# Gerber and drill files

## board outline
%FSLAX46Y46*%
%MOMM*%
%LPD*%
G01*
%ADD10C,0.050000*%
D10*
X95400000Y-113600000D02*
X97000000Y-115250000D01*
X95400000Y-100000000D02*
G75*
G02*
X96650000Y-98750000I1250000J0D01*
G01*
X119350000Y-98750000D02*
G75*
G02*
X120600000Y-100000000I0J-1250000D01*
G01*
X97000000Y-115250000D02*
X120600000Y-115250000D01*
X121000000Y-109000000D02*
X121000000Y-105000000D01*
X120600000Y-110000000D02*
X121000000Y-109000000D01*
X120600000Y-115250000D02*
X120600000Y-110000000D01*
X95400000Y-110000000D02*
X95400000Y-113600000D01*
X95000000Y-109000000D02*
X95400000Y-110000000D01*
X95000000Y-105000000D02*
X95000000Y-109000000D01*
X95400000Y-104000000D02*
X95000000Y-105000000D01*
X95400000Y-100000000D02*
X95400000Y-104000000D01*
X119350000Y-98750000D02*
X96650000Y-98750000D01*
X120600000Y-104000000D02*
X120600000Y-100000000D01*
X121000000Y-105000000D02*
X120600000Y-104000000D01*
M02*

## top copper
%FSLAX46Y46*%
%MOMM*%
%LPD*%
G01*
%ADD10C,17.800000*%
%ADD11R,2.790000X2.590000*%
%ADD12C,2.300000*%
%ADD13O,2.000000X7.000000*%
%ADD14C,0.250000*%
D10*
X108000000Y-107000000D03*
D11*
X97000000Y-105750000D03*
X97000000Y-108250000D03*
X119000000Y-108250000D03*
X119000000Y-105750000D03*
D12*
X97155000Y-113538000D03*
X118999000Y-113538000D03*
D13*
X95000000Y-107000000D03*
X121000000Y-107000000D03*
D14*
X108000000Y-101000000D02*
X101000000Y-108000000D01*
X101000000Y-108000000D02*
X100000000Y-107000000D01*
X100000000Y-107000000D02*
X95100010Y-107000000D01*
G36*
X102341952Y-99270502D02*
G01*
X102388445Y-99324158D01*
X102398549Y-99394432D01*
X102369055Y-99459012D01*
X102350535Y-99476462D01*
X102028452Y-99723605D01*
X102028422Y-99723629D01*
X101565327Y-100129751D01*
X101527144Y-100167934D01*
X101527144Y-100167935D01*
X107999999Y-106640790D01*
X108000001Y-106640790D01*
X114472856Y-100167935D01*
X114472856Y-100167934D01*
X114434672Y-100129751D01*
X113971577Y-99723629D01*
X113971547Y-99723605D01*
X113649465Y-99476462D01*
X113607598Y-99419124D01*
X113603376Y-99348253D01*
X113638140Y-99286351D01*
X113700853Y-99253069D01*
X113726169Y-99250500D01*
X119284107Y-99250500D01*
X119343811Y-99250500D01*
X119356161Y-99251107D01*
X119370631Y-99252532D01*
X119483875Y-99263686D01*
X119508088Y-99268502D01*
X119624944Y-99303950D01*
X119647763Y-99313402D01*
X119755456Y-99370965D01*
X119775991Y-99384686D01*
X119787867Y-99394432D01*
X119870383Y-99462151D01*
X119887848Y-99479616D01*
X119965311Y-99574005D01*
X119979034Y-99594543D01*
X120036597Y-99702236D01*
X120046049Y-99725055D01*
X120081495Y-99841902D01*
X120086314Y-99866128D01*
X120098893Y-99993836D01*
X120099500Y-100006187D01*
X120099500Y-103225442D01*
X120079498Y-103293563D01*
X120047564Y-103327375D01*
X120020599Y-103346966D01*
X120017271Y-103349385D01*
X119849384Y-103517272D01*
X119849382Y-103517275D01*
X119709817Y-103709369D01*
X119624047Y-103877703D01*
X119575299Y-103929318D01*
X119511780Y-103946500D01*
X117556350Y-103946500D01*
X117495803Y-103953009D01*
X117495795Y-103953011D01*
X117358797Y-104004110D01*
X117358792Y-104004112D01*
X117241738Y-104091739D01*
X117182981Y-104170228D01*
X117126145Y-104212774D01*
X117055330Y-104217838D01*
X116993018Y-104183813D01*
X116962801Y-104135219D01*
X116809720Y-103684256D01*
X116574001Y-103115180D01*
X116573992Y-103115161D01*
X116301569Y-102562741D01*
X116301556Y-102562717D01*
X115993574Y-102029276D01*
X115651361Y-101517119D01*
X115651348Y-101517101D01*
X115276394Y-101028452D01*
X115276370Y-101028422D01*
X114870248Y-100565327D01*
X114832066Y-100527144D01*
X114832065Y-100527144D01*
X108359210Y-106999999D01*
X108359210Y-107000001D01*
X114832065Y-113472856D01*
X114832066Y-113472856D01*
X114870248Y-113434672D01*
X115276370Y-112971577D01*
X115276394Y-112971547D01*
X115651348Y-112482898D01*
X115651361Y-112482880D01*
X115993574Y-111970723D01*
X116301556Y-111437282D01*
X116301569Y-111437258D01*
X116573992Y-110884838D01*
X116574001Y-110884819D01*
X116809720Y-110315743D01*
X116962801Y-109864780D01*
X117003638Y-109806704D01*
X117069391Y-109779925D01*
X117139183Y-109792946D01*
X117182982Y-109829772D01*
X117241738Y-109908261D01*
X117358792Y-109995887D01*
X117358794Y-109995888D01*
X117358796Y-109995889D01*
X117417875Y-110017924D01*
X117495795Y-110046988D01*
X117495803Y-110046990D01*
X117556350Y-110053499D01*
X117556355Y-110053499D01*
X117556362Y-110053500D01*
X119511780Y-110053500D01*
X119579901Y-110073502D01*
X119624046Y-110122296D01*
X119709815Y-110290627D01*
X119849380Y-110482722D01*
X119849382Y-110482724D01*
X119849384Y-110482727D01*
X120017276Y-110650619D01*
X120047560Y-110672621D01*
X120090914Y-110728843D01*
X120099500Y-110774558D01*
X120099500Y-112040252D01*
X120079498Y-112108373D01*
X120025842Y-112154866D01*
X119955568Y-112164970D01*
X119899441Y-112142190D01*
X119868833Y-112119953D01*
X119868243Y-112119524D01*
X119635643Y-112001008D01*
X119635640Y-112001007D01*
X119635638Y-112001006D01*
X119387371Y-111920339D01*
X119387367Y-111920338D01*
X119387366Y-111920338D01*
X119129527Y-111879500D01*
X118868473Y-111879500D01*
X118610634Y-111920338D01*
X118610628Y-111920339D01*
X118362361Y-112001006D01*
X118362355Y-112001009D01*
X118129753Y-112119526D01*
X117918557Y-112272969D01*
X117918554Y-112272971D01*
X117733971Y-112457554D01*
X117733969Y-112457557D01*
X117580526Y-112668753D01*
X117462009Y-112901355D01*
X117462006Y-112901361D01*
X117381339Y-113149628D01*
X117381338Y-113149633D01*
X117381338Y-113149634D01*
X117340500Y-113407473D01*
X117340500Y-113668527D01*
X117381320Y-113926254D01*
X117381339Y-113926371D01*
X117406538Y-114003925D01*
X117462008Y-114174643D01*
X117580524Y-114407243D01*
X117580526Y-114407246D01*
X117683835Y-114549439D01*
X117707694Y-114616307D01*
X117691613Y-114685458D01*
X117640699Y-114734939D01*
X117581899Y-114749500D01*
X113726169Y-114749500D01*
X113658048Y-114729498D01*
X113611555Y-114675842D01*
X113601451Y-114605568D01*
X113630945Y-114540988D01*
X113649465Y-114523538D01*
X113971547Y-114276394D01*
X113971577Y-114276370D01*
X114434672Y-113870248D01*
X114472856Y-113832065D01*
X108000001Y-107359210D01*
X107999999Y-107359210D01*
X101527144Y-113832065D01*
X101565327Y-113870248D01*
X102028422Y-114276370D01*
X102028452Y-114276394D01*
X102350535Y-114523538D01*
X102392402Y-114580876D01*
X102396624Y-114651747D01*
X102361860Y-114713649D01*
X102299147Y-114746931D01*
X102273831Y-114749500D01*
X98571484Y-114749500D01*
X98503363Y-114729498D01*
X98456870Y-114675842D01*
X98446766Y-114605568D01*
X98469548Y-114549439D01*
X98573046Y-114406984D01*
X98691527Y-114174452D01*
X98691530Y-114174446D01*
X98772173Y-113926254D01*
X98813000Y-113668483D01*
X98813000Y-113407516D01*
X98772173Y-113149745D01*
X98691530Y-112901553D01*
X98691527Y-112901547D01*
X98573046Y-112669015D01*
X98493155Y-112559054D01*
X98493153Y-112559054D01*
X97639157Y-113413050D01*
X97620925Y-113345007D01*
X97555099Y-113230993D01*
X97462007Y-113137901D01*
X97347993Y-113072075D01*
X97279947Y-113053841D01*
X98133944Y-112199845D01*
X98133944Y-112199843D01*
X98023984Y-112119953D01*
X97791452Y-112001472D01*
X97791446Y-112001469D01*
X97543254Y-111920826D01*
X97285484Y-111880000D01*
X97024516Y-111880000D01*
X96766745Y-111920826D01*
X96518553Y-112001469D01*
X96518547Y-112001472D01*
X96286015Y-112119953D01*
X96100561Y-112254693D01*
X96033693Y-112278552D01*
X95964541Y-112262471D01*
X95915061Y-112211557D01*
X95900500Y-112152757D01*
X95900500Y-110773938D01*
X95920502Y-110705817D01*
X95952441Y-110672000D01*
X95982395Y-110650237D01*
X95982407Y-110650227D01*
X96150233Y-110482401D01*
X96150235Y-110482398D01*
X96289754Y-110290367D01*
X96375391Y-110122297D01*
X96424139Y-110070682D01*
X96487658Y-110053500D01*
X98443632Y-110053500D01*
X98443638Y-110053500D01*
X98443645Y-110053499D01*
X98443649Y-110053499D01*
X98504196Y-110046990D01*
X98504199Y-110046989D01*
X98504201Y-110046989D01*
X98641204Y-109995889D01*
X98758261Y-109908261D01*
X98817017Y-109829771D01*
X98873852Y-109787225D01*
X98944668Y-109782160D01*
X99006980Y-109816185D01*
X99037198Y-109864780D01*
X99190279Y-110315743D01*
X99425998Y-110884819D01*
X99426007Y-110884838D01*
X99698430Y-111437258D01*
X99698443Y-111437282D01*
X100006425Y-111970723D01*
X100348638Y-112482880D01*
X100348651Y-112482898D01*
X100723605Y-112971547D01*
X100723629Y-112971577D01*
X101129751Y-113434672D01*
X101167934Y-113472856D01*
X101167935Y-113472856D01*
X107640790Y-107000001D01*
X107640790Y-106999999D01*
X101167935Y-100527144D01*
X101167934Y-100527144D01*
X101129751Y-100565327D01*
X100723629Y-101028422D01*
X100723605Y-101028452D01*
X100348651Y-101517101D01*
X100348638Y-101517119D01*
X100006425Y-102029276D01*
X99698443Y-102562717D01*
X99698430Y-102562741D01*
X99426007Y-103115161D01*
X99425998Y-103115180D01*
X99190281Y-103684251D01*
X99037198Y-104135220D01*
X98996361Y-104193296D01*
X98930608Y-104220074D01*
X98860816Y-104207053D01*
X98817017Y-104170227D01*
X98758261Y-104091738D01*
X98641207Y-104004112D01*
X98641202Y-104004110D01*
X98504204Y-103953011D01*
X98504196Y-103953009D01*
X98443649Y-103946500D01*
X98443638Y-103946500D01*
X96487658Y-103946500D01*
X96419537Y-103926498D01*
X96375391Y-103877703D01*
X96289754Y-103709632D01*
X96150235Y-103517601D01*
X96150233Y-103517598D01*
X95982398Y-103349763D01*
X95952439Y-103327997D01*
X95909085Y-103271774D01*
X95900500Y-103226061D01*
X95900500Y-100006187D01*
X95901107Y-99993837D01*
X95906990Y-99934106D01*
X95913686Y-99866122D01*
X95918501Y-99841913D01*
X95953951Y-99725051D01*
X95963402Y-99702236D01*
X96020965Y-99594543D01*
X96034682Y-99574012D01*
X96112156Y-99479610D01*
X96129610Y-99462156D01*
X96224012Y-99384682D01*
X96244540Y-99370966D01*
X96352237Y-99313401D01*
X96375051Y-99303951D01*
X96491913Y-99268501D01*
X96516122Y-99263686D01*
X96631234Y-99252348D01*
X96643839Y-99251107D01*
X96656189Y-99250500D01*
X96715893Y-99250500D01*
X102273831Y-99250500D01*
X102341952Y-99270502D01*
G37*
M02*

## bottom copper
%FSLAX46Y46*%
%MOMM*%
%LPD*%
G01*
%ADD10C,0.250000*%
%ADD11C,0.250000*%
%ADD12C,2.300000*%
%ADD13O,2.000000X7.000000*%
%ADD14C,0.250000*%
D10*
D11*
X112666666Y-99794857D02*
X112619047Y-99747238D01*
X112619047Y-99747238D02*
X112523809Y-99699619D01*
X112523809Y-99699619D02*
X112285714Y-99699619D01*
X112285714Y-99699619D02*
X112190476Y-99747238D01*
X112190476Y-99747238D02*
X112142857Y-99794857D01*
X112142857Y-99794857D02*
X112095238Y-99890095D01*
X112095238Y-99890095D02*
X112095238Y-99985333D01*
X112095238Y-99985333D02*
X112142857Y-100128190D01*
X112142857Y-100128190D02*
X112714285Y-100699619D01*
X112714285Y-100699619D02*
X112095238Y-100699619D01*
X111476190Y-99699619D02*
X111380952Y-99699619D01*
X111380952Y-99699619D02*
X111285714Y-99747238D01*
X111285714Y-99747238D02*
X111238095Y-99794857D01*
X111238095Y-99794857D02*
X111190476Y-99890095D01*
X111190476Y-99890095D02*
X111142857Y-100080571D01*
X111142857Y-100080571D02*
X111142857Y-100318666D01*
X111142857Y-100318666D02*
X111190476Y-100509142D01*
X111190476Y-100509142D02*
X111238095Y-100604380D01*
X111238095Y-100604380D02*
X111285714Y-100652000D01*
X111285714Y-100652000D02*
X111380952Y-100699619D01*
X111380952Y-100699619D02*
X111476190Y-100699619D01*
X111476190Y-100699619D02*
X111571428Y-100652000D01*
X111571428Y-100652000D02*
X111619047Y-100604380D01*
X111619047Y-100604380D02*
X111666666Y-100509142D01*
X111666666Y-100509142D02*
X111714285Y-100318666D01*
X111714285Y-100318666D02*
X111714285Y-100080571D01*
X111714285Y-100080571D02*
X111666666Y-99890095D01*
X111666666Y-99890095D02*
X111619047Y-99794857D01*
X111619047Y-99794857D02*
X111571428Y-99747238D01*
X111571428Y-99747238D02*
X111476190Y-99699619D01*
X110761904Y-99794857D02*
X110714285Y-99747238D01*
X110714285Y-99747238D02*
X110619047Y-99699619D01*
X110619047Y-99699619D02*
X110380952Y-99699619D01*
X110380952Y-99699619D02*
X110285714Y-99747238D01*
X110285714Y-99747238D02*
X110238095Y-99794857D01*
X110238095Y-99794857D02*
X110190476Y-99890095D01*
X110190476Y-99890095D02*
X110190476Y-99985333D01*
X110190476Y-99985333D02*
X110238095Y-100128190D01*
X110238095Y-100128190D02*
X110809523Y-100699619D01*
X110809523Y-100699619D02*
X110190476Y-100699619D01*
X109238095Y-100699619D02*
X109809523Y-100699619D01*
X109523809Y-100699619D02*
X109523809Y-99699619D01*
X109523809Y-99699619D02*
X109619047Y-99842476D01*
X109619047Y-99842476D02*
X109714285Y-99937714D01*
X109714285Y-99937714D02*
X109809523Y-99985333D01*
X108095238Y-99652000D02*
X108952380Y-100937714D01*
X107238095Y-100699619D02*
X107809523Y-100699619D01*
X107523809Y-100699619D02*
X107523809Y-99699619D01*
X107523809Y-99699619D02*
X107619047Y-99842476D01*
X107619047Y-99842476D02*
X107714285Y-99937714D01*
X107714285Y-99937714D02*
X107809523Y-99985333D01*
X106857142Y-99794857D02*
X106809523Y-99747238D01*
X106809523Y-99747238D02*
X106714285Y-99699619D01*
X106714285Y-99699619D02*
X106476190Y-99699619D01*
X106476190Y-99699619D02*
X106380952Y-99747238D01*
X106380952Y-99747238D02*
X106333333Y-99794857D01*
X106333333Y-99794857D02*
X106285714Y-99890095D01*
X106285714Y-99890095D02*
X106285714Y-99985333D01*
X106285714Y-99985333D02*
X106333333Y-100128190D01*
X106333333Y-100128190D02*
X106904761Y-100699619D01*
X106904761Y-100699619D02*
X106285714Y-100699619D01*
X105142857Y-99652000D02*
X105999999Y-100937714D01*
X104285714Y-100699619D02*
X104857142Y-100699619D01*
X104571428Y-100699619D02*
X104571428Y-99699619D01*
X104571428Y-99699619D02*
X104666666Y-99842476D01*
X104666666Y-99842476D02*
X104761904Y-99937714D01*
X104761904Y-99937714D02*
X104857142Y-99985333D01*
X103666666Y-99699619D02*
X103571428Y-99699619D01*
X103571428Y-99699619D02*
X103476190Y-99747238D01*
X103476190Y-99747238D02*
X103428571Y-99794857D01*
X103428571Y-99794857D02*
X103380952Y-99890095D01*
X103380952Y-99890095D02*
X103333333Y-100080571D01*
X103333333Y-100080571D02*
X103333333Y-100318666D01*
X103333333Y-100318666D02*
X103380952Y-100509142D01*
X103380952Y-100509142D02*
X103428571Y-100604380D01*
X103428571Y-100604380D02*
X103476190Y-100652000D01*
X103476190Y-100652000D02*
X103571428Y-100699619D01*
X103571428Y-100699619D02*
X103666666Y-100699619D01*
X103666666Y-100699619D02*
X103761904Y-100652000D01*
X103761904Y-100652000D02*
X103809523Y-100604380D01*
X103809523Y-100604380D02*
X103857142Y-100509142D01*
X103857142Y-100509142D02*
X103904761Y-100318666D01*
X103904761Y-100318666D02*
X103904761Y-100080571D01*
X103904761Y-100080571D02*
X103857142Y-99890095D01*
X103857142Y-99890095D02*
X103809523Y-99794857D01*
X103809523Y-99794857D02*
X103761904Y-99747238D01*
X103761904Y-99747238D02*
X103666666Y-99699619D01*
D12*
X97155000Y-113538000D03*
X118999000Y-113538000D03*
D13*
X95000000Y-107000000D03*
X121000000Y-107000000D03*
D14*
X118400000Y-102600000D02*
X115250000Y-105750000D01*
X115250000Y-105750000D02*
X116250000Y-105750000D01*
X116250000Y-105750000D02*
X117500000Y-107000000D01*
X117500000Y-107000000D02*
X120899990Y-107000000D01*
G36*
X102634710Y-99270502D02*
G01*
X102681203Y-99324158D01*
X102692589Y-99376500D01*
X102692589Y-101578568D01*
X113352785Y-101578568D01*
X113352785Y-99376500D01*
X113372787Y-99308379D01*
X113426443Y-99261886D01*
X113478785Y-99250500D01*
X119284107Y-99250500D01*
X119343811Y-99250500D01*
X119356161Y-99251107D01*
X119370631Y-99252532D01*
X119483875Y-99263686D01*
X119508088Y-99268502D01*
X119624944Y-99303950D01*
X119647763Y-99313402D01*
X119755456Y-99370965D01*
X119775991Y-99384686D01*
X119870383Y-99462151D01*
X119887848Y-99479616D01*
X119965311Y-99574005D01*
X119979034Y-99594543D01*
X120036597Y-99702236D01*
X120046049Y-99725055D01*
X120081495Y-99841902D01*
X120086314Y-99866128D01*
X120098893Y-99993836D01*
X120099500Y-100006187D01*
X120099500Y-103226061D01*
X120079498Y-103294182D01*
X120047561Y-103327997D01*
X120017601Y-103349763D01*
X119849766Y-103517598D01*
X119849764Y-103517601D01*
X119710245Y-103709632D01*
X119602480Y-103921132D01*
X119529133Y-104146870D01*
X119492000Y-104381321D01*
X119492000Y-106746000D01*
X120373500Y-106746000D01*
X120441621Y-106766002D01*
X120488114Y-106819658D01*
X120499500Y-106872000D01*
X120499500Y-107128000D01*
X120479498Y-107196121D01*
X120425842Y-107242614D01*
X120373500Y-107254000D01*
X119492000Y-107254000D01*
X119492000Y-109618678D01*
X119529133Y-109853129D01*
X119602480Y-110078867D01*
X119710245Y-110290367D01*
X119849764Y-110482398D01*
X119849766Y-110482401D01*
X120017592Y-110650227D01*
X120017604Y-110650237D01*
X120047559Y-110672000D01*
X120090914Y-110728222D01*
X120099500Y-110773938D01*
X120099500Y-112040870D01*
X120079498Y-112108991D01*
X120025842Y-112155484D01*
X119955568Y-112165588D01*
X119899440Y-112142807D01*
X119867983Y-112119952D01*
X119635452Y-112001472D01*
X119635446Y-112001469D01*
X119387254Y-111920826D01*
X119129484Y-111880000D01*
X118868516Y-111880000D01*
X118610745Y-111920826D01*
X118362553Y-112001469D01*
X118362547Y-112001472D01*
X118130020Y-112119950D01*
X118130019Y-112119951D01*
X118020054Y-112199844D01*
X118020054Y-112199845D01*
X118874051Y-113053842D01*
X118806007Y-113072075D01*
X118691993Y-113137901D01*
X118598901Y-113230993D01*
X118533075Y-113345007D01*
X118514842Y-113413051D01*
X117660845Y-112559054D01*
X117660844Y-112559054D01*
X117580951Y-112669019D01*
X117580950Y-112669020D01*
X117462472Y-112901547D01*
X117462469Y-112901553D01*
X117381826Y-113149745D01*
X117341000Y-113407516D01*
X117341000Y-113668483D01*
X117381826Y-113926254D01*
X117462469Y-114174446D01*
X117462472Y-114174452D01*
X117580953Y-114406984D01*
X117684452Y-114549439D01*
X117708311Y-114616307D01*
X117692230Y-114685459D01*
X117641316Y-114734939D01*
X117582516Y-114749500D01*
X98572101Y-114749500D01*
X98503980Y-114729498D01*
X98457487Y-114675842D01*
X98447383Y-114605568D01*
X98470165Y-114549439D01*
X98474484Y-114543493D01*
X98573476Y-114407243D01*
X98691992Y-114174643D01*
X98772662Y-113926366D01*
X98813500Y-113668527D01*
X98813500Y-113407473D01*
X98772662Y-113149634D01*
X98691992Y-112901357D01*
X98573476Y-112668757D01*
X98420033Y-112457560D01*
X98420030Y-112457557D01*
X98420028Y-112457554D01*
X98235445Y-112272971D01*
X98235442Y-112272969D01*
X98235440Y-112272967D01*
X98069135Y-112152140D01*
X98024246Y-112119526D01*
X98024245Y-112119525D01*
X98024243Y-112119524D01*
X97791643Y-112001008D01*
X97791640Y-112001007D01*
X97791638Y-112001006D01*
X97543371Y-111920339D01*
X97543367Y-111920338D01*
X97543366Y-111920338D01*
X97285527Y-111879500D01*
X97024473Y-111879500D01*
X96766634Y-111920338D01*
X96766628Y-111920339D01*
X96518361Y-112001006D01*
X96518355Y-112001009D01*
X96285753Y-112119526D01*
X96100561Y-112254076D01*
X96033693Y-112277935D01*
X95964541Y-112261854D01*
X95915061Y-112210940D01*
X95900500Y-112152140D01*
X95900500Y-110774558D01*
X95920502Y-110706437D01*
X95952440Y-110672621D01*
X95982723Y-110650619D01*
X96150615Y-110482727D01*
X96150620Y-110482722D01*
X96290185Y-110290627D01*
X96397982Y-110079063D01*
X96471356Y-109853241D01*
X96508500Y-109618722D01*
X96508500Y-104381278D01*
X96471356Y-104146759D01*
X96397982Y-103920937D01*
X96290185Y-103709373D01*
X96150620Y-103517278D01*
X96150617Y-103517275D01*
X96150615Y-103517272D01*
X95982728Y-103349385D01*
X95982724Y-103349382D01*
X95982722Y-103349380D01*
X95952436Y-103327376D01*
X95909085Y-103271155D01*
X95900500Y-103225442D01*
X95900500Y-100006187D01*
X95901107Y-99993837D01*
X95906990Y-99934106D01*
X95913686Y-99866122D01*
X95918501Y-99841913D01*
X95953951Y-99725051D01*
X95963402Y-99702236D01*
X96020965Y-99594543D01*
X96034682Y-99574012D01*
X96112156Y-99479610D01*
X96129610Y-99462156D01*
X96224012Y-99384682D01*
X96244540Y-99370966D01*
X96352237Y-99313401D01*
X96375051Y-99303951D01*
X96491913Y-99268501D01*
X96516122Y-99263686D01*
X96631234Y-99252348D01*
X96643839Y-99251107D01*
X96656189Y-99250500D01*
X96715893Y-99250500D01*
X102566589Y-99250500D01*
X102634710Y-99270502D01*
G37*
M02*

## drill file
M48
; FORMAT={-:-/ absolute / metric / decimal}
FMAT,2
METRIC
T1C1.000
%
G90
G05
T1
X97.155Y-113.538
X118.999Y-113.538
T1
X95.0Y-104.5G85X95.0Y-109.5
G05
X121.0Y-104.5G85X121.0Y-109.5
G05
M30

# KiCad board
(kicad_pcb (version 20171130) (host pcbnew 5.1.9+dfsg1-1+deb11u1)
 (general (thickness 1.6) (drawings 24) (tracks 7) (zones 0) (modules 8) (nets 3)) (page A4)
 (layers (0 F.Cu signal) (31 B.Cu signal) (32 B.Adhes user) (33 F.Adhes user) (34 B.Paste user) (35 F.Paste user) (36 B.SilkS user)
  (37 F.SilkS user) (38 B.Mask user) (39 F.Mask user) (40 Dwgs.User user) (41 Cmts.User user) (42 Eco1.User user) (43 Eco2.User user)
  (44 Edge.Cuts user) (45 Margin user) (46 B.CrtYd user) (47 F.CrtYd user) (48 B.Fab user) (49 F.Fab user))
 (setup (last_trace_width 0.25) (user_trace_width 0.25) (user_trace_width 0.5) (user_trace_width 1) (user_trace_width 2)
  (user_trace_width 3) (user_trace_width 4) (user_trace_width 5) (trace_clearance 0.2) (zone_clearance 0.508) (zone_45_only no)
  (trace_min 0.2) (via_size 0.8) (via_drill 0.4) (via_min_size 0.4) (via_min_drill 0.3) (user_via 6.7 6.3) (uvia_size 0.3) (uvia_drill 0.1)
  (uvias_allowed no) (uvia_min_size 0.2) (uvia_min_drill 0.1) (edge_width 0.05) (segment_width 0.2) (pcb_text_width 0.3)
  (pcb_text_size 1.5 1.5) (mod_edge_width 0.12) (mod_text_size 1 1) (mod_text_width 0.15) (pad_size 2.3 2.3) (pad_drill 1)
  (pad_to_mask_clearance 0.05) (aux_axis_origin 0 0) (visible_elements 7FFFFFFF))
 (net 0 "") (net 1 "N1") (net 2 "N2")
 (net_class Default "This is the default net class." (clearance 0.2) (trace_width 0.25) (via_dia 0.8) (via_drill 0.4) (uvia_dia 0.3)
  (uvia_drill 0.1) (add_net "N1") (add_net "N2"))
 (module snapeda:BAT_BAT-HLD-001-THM (layer F.Cu) (at 108 107)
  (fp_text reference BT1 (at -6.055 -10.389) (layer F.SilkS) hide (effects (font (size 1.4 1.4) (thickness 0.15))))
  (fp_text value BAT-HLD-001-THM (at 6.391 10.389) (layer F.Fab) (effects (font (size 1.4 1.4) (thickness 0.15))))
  (pad N smd circle (at 0 0) (size 17.8 17.8) (layers F.Cu F.Mask) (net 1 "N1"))
  (pad P1 smd rect (at -11 -1.25) (size 2.79 2.59) (layers F.Cu F.Paste F.Mask) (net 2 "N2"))
  (pad P2 smd rect (at -11 1.25) (size 2.79 2.59) (layers F.Cu F.Paste F.Mask) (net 2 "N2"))
  (pad P3 smd rect (at 11 1.25) (size 2.79 2.59) (layers F.Cu F.Paste F.Mask) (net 2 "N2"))
  (pad P4 smd rect (at 11 -1.25) (size 2.79 2.59) (layers F.Cu F.Paste F.Mask) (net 2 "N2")))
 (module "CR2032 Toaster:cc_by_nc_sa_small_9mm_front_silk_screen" (layer B.Cu) (at 107.95 113.5 180)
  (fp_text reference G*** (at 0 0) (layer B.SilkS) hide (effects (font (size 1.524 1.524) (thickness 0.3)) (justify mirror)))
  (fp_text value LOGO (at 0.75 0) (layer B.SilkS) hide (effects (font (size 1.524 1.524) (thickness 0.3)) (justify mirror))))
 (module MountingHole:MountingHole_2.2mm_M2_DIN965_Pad (layer F.Cu) (at 97.155 113.538)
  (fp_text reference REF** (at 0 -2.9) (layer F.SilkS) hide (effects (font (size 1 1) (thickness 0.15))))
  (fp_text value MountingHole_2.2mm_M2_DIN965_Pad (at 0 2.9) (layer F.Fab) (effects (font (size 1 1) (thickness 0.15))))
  (pad 1 thru_hole circle (at 0 0) (size 2.3 2.3) (drill 1) (layers *.Cu *.Mask) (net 1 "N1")))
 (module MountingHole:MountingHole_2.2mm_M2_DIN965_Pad (layer F.Cu) (at 118.999 113.538)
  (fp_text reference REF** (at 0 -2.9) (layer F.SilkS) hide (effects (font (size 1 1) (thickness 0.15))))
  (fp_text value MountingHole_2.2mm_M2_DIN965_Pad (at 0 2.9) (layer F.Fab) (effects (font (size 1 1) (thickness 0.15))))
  (pad 1 thru_hole circle (at 0 0) (size 2.3 2.3) (drill 1) (layers *.Cu *.Mask) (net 2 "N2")))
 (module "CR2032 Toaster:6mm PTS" (layer F.Cu) (at 95 107)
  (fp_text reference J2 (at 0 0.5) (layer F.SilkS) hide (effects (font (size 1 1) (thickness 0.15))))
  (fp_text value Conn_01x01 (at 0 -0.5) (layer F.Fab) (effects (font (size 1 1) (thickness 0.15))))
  (pad 1 thru_hole oval (at 0 0) (size 2 7) (drill oval 1 6) (layers *.Cu *.Mask) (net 1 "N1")))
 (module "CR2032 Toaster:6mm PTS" (layer F.Cu) (at 121 107)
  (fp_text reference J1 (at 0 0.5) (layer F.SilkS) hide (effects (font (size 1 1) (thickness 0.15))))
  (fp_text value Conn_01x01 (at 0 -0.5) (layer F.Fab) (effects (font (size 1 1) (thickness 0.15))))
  (pad 1 thru_hole oval (at 0 0) (size 2 7) (drill oval 1 6) (layers *.Cu *.Mask) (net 2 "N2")))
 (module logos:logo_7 (layer F.Cu) (at 114 106.25)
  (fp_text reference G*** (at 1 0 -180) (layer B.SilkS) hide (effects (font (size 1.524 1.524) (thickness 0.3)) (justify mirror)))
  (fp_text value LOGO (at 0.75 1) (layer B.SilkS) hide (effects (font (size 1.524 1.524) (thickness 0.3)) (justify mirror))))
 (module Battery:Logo (layer F.Cu) (at 0 0)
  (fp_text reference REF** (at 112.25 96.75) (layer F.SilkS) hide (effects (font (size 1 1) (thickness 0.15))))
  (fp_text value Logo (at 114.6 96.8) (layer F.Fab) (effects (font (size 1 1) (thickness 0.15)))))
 (gr_line (start 95.4 113.6) (end 97 115.25) (layer Edge.Cuts) (width 0.05))
 (gr_arc (start 96.65 100) (end 96.65 98.75) (angle -90) (layer Edge.Cuts) (width 0.05))
 (gr_arc (start 119.35 100) (end 120.6 100) (angle -90) (layer Edge.Cuts) (width 0.05))
 (gr_line (start 97 115.25) (end 120.6 115.25) (layer Edge.Cuts) (width 0.05))
 (gr_line (start 121 109) (end 121 105) (layer Edge.Cuts) (width 0.05))
 (gr_line (start 120.6 110) (end 121 109) (layer Edge.Cuts) (width 0.05))
 (gr_line (start 120.6 115.25) (end 120.6 110) (layer Edge.Cuts) (width 0.05))
 (gr_line (start 95.4 110) (end 95.4 113.6) (layer Edge.Cuts) (width 0.05))
 (gr_line (start 95 109) (end 95.4 110) (layer Edge.Cuts) (width 0.05))
 (gr_line (start 95 105) (end 95 109) (layer Edge.Cuts) (width 0.05))
 (gr_line (start 95.4 104) (end 95 105) (layer Edge.Cuts) (width 0.05))
 (gr_line (start 95.4 100) (end 95.4 104) (layer Edge.Cuts) (width 0.05))
 (gr_line (start 119.35 98.75) (end 96.65 98.75) (layer Edge.Cuts) (width 0.05))
 (gr_line (start 120.6 104) (end 120.6 100) (layer Edge.Cuts) (width 0.05))
 (gr_line (start 121 105) (end 120.6 104) (layer Edge.Cuts) (width 0.05))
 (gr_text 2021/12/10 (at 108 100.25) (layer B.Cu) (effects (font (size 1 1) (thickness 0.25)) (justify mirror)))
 (segment (start 118.4 102.6) (end 115.25 105.75) (width 0.25) (layer B.Cu) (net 2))
 (segment (start 115.25 105.75) (end 116.25 105.75) (width 0.25) (layer B.Cu) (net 2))
 (segment (start 116.25 105.75) (end 117.5 107) (width 0.25) (layer B.Cu) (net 2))
 (segment (start 117.5 107) (end 120.89999 107) (width 0.25) (layer B.Cu) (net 2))
 (segment (start 108 101) (end 101 108) (width 0.25) (layer F.Cu) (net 1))
 (segment (start 101 108) (end 100 107) (width 0.25) (layer F.Cu) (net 1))
 (segment (start 100 107) (end 95.10001 107) (width 0.25) (layer F.Cu) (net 1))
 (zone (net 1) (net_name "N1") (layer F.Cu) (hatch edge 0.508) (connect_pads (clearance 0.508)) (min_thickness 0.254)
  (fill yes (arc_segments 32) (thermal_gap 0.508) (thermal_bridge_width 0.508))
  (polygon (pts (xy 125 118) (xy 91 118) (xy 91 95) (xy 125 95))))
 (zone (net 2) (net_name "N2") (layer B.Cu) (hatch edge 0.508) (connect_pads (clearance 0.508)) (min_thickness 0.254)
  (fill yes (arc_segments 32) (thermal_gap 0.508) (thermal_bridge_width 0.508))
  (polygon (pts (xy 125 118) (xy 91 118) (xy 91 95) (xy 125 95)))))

